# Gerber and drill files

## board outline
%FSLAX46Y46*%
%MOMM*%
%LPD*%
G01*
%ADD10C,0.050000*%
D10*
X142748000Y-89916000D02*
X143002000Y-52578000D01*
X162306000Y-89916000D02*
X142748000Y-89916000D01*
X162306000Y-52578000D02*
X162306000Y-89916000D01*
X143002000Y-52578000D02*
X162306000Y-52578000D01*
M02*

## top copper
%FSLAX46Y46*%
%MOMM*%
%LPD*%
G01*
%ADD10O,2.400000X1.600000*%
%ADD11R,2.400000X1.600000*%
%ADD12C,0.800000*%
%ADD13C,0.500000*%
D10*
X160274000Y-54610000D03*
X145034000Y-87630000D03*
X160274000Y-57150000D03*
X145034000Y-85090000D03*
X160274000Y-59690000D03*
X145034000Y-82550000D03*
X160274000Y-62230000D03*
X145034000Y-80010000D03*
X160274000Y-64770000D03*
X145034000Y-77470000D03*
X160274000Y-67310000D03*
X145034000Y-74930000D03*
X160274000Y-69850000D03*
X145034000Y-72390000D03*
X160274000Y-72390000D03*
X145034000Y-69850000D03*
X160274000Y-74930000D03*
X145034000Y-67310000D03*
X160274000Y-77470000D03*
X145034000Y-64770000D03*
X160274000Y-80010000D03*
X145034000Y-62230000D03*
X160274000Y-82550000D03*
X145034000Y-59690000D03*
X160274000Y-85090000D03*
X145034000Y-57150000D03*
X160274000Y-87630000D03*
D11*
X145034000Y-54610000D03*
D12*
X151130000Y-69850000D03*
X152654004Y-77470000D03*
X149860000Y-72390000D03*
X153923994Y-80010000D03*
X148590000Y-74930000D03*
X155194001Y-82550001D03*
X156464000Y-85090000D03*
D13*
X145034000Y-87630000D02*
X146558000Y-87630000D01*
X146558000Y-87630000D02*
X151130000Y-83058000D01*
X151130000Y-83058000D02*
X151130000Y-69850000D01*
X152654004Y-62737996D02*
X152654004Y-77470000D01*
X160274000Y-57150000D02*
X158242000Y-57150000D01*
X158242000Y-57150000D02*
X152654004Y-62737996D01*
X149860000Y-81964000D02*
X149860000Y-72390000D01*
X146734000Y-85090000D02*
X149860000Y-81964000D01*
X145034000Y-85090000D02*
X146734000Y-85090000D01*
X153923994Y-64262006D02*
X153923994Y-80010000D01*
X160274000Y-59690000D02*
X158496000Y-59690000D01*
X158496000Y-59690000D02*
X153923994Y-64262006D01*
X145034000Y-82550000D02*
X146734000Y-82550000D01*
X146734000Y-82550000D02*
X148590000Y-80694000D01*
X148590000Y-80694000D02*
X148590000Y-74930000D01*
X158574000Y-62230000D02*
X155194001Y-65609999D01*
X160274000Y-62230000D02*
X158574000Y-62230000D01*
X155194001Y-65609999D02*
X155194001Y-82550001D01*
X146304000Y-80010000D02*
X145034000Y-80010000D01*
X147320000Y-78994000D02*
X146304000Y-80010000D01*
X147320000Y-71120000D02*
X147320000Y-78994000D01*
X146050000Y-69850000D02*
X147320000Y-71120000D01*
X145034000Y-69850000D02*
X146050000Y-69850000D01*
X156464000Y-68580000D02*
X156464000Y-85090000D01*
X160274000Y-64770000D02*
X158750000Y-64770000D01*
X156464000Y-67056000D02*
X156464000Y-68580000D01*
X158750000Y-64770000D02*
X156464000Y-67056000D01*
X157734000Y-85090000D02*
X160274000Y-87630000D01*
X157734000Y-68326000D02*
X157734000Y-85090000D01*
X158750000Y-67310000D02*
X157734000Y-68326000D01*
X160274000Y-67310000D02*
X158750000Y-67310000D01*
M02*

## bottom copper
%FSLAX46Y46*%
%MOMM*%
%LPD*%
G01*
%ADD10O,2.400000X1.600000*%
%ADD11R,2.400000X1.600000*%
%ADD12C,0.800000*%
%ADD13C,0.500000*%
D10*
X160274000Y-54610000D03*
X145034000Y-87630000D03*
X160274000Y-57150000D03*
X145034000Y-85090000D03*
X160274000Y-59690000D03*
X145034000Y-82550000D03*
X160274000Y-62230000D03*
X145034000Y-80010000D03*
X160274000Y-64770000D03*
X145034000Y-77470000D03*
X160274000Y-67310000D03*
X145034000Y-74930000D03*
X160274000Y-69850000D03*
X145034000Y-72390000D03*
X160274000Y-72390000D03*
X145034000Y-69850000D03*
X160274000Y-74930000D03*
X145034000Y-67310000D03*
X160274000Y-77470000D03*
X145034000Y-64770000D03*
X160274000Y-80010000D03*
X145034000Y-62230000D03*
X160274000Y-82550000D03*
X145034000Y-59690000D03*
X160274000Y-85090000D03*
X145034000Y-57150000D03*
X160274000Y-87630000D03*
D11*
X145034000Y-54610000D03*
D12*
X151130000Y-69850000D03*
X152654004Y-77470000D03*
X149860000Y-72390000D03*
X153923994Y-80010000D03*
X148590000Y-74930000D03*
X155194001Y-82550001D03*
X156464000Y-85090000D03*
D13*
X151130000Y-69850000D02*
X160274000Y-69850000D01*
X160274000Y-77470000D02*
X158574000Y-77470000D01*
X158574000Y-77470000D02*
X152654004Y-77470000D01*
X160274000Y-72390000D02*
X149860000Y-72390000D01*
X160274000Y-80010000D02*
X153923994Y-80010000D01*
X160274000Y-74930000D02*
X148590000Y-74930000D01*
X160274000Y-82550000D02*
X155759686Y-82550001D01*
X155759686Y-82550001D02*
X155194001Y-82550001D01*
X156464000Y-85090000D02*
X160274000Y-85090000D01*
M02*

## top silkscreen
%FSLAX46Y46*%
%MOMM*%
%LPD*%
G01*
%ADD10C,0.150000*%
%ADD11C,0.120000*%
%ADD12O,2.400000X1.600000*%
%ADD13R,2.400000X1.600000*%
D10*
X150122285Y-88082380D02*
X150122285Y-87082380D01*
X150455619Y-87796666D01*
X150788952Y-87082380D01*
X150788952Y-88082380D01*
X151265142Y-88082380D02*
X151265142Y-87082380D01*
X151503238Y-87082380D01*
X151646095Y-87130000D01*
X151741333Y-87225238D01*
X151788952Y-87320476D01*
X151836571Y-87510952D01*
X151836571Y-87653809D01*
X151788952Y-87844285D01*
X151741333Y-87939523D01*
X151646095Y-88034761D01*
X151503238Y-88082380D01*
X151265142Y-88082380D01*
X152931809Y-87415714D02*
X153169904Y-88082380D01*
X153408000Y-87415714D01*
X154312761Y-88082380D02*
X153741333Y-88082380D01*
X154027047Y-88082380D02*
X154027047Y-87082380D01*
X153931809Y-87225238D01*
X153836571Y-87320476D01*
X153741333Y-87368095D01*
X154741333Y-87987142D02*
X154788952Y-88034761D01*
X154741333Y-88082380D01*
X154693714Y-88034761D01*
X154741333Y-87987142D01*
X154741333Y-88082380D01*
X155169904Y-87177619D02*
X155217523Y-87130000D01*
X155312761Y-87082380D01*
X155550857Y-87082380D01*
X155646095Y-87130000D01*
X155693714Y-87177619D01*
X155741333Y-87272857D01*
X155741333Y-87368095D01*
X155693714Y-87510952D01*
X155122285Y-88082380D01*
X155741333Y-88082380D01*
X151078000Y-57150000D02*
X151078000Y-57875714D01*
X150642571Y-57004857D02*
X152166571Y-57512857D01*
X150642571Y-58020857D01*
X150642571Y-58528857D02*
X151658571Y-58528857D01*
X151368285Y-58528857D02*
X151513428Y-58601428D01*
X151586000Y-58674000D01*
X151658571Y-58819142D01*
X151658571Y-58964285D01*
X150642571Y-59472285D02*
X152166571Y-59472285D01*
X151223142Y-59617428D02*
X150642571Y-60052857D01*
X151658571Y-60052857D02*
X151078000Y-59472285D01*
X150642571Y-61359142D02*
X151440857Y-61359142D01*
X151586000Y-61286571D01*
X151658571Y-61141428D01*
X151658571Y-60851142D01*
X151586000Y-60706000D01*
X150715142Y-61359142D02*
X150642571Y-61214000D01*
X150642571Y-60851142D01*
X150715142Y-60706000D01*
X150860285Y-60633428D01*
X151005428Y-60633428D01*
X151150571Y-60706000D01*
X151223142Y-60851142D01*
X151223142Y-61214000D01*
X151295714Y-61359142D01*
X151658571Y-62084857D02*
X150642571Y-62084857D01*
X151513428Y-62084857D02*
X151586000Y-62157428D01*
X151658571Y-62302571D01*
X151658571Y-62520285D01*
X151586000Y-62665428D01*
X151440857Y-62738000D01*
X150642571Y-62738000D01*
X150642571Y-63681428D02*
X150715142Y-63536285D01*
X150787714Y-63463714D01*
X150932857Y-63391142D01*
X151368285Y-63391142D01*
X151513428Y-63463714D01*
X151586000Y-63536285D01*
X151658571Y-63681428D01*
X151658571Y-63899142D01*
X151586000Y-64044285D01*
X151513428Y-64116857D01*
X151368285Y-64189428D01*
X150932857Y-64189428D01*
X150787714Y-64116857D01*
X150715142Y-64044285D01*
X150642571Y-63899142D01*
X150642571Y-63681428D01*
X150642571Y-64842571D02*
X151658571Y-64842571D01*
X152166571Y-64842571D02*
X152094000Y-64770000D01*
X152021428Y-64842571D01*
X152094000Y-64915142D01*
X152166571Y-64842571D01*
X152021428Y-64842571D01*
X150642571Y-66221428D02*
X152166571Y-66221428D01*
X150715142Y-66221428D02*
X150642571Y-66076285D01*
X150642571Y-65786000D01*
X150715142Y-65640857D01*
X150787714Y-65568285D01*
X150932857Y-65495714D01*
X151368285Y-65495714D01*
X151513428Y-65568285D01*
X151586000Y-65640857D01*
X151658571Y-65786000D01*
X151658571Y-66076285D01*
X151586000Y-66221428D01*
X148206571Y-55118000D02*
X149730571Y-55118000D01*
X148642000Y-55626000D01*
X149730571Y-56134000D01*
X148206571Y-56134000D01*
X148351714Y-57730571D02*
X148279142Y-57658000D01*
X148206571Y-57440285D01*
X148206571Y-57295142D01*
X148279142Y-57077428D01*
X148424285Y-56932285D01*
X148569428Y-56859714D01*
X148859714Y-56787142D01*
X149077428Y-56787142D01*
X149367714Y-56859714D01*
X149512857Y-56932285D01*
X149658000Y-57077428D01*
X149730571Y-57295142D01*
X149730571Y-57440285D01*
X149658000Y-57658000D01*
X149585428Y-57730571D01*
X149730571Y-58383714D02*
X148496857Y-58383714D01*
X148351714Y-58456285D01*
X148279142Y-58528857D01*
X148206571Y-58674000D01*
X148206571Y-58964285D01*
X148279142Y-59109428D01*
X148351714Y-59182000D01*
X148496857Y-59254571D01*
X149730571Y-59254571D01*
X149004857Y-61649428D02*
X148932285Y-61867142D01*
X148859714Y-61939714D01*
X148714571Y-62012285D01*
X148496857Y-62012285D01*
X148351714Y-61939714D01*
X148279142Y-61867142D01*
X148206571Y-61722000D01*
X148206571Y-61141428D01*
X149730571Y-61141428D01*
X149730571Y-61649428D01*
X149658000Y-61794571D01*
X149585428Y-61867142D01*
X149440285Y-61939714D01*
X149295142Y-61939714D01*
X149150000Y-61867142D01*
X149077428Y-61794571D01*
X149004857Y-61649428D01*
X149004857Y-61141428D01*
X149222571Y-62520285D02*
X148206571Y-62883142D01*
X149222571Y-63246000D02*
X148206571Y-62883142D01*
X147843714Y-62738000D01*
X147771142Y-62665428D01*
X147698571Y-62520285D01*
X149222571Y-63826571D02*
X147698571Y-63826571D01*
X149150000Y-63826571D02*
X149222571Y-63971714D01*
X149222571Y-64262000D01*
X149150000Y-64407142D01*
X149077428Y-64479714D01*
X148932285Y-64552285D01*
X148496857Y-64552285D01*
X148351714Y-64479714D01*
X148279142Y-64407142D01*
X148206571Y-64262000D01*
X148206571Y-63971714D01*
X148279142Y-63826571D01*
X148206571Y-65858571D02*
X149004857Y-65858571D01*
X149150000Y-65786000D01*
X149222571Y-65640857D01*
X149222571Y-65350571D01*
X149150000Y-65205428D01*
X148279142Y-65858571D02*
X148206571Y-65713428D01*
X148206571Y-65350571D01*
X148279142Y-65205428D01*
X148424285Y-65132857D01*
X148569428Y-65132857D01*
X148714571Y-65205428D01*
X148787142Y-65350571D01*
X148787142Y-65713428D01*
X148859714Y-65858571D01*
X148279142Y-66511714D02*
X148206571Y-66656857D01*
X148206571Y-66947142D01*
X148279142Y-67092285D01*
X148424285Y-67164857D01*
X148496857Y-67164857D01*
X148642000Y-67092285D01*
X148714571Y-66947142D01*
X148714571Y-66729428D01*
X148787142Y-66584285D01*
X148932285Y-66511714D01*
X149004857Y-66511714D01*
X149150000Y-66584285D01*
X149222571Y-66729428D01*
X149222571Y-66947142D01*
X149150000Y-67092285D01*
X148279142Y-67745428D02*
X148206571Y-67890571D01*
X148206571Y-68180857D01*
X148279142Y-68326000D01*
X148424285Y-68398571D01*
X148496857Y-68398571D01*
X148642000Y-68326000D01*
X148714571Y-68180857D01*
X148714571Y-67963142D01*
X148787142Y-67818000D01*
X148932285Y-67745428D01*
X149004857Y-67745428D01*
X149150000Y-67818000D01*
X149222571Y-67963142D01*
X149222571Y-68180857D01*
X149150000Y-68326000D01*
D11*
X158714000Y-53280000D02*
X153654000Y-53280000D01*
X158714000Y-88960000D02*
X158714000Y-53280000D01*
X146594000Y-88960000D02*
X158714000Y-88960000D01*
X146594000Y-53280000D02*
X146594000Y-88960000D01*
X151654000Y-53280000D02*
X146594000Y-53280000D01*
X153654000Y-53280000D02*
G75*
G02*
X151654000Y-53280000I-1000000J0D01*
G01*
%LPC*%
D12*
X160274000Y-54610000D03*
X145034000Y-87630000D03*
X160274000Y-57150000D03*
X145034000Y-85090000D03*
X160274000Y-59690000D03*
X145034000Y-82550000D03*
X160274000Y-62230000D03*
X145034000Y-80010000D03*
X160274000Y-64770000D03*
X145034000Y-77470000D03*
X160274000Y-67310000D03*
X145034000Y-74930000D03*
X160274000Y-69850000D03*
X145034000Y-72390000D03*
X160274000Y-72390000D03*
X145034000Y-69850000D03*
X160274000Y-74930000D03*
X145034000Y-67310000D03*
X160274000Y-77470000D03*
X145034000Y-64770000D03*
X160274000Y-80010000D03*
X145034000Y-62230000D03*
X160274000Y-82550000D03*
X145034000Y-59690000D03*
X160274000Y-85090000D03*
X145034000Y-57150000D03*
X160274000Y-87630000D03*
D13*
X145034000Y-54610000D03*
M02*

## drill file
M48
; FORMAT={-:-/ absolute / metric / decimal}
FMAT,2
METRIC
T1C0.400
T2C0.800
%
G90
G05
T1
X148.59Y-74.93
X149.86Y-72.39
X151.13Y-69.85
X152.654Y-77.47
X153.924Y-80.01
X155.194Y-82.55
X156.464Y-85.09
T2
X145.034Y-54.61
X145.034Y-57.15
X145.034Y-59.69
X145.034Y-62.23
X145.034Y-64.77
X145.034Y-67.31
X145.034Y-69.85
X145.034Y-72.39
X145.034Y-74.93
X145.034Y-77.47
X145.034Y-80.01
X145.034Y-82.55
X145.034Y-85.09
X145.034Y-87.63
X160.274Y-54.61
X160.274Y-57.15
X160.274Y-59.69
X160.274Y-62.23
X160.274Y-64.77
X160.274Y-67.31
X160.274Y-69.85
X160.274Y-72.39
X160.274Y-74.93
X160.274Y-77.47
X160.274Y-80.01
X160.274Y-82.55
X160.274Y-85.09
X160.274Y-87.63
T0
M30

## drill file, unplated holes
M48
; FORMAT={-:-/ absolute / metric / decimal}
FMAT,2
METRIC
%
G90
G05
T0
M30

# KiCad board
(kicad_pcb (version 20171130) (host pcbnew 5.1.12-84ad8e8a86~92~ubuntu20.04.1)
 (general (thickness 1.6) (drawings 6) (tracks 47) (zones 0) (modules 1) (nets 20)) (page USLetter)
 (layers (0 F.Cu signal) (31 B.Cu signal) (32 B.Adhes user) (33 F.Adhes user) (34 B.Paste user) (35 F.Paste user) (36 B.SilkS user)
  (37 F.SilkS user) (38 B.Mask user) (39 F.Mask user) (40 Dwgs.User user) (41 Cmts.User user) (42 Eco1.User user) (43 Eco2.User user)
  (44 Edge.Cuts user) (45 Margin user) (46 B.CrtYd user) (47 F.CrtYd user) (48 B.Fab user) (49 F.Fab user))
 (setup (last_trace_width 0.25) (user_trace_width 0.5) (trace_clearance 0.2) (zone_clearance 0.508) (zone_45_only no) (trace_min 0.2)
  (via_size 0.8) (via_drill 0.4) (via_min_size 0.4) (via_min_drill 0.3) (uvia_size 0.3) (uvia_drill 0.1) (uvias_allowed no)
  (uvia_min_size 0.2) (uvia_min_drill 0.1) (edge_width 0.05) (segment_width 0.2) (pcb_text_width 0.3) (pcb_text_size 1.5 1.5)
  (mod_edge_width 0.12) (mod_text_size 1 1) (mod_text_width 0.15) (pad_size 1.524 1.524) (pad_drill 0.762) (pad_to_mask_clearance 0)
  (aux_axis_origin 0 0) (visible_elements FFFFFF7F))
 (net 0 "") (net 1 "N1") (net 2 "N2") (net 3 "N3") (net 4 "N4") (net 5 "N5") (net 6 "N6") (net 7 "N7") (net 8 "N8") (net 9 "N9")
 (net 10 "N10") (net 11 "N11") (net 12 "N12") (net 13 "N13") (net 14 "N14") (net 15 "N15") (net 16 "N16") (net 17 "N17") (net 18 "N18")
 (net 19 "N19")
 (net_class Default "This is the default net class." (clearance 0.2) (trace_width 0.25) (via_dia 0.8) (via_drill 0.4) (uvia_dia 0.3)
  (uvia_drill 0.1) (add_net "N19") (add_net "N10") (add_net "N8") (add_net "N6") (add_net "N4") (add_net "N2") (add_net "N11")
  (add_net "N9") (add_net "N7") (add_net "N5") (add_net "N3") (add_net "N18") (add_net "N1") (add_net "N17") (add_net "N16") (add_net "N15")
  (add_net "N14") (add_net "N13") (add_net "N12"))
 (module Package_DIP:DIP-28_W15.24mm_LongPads (layer F.Cu) (at 145.034 54.61)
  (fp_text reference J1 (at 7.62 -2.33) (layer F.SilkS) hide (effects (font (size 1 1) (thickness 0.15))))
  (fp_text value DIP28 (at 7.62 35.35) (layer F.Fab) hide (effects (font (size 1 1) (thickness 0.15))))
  (fp_line (start 6.62 -1.33) (end 1.56 -1.33) (layer F.SilkS) (width 0.12))
  (fp_line (start 1.56 -1.33) (end 1.56 34.35) (layer F.SilkS) (width 0.12))
  (fp_line (start 1.56 34.35) (end 13.68 34.35) (layer F.SilkS) (width 0.12))
  (fp_line (start 13.68 34.35) (end 13.68 -1.33) (layer F.SilkS) (width 0.12))
  (fp_line (start 13.68 -1.33) (end 8.62 -1.33) (layer F.SilkS) (width 0.12))
  (fp_arc (start 7.62 -1.33) (end 6.62 -1.33) (angle -180) (layer F.SilkS) (width 0.12))
  (pad 28 thru_hole oval (at 15.24 0) (size 2.4 1.6) (drill 0.8) (layers *.Cu *.Mask) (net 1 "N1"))
  (pad 14 thru_hole oval (at 0 33.02) (size 2.4 1.6) (drill 0.8) (layers *.Cu *.Mask) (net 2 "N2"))
  (pad 27 thru_hole oval (at 15.24 2.54) (size 2.4 1.6) (drill 0.8) (layers *.Cu *.Mask) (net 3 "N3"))
  (pad 13 thru_hole oval (at 0 30.48) (size 2.4 1.6) (drill 0.8) (layers *.Cu *.Mask) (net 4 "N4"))
  (pad 26 thru_hole oval (at 15.24 5.08) (size 2.4 1.6) (drill 0.8) (layers *.Cu *.Mask) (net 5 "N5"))
  (pad 12 thru_hole oval (at 0 27.94) (size 2.4 1.6) (drill 0.8) (layers *.Cu *.Mask) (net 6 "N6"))
  (pad 25 thru_hole oval (at 15.24 7.62) (size 2.4 1.6) (drill 0.8) (layers *.Cu *.Mask) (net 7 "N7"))
  (pad 11 thru_hole oval (at 0 25.4) (size 2.4 1.6) (drill 0.8) (layers *.Cu *.Mask) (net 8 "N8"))
  (pad 24 thru_hole oval (at 15.24 10.16) (size 2.4 1.6) (drill 0.8) (layers *.Cu *.Mask) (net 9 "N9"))
  (pad 10 thru_hole oval (at 0 22.86) (size 2.4 1.6) (drill 0.8) (layers *.Cu *.Mask) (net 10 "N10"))
  (pad 23 thru_hole oval (at 15.24 12.7) (size 2.4 1.6) (drill 0.8) (layers *.Cu *.Mask) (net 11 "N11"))
  (pad 9 thru_hole oval (at 0 20.32) (size 2.4 1.6) (drill 0.8) (layers *.Cu *.Mask) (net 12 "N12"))
  (pad 22 thru_hole oval (at 15.24 15.24) (size 2.4 1.6) (drill 0.8) (layers *.Cu *.Mask) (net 2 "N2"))
  (pad 8 thru_hole oval (at 0 17.78) (size 2.4 1.6) (drill 0.8) (layers *.Cu *.Mask) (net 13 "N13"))
  (pad 21 thru_hole oval (at 15.24 17.78) (size 2.4 1.6) (drill 0.8) (layers *.Cu *.Mask) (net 4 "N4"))
  (pad 7 thru_hole oval (at 0 15.24) (size 2.4 1.6) (drill 0.8) (layers *.Cu *.Mask) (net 8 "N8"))
  (pad 20 thru_hole oval (at 15.24 20.32) (size 2.4 1.6) (drill 0.8) (layers *.Cu *.Mask) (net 6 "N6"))
  (pad 6 thru_hole oval (at 0 12.7) (size 2.4 1.6) (drill 0.8) (layers *.Cu *.Mask) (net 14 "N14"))
  (pad 19 thru_hole oval (at 15.24 22.86) (size 2.4 1.6) (drill 0.8) (layers *.Cu *.Mask) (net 3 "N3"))
  (pad 5 thru_hole oval (at 0 10.16) (size 2.4 1.6) (drill 0.8) (layers *.Cu *.Mask) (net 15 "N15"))
  (pad 18 thru_hole oval (at 15.24 25.4) (size 2.4 1.6) (drill 0.8) (layers *.Cu *.Mask) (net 5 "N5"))
  (pad 4 thru_hole oval (at 0 7.62) (size 2.4 1.6) (drill 0.8) (layers *.Cu *.Mask) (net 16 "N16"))
  (pad 17 thru_hole oval (at 15.24 27.94) (size 2.4 1.6) (drill 0.8) (layers *.Cu *.Mask) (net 7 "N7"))
  (pad 3 thru_hole oval (at 0 5.08) (size 2.4 1.6) (drill 0.8) (layers *.Cu *.Mask) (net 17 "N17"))
  (pad 16 thru_hole oval (at 15.24 30.48) (size 2.4 1.6) (drill 0.8) (layers *.Cu *.Mask) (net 9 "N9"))
  (pad 2 thru_hole oval (at 0 2.54) (size 2.4 1.6) (drill 0.8) (layers *.Cu *.Mask) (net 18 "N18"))
  (pad 15 thru_hole oval (at 15.24 33.02) (size 2.4 1.6) (drill 0.8) (layers *.Cu *.Mask) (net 11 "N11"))
  (pad 1 thru_hole rect (at 0 0) (size 2.4 1.6) (drill 0.8) (layers *.Cu *.Mask) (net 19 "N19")))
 (gr_line (start 142.748 89.916) (end 143.002 52.578) (layer Edge.Cuts) (width 0.05))
 (gr_line (start 162.306 89.916) (end 142.748 89.916) (layer Edge.Cuts) (width 0.05))
 (gr_line (start 162.306 52.578) (end 162.306 89.916) (layer Edge.Cuts) (width 0.05))
 (gr_line (start 143.002 52.578) (end 162.306 52.578) (layer Edge.Cuts) (width 0.05))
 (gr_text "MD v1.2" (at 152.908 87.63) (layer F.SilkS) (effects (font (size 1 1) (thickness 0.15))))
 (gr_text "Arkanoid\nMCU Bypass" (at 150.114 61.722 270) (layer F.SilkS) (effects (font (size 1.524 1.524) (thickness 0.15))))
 (segment (start 145.034 87.63) (end 146.558 87.63) (width 0.5) (layer F.Cu) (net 2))
 (segment (start 146.558 87.63) (end 151.13 83.058) (width 0.5) (layer F.Cu) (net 2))
 (segment (start 151.13 83.058) (end 151.13 69.85) (width 0.5) (layer F.Cu) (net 2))
 (via (at 151.13 69.85) (size 0.8) (drill 0.4) (layers F.Cu B.Cu) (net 2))
 (segment (start 151.13 69.85) (end 160.274 69.85) (width 0.5) (layer B.Cu) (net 2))
 (via (at 152.654004 77.47) (size 0.8) (drill 0.4) (layers F.Cu B.Cu) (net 3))
 (segment (start 160.274 77.47) (end 158.574 77.47) (width 0.5) (layer B.Cu) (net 3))
 (segment (start 152.654004 62.737996) (end 152.654004 77.47) (width 0.5) (layer F.Cu) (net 3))
 (segment (start 158.574 77.47) (end 152.654004 77.47) (width 0.5) (layer B.Cu) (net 3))
 (segment (start 160.274 57.15) (end 158.242 57.15) (width 0.5) (layer F.Cu) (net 3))
 (segment (start 158.242 57.15) (end 152.654004 62.737996) (width 0.5) (layer F.Cu) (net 3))
 (segment (start 149.86 81.964) (end 149.86 72.39) (width 0.5) (layer F.Cu) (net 4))
 (segment (start 146.734 85.09) (end 149.86 81.964) (width 0.5) (layer F.Cu) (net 4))
 (segment (start 145.034 85.09) (end 146.734 85.09) (width 0.5) (layer F.Cu) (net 4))
 (segment (start 160.274 72.39) (end 149.86 72.39) (width 0.5) (layer B.Cu) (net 4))
 (via (at 149.86 72.39) (size 0.8) (drill 0.4) (layers F.Cu B.Cu) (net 4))
 (via (at 153.923994 80.01) (size 0.8) (drill 0.4) (layers F.Cu B.Cu) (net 5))
 (segment (start 160.274 80.01) (end 153.923994 80.01) (width 0.5) (layer B.Cu) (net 5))
 (segment (start 153.923994 64.262006) (end 153.923994 80.01) (width 0.5) (layer F.Cu) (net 5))
 (segment (start 160.274 59.69) (end 158.496 59.69) (width 0.5) (layer F.Cu) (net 5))
 (segment (start 158.496 59.69) (end 153.923994 64.262006) (width 0.5) (layer F.Cu) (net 5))
 (via (at 148.59 74.93) (size 0.8) (drill 0.4) (layers F.Cu B.Cu) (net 6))
 (segment (start 160.274 74.93) (end 148.59 74.93) (width 0.5) (layer B.Cu) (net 6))
 (segment (start 145.034 82.55) (end 146.734 82.55) (width 0.5) (layer F.Cu) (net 6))
 (segment (start 146.734 82.55) (end 148.59 80.694) (width 0.5) (layer F.Cu) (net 6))
 (segment (start 148.59 80.694) (end 148.59 74.93) (width 0.5) (layer F.Cu) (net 6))
 (via (at 155.194001 82.550001) (size 0.8) (drill 0.4) (layers F.Cu B.Cu) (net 7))
 (segment (start 160.274 82.55) (end 155.759686 82.550001) (width 0.5) (layer B.Cu) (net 7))
 (segment (start 155.759686 82.550001) (end 155.194001 82.550001) (width 0.5) (layer B.Cu) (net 7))
 (segment (start 158.574 62.23) (end 155.194001 65.609999) (width 0.5) (layer F.Cu) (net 7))
 (segment (start 160.274 62.23) (end 158.574 62.23) (width 0.5) (layer F.Cu) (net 7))
 (segment (start 155.194001 65.609999) (end 155.194001 82.550001) (width 0.5) (layer F.Cu) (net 7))
 (segment (start 146.304 80.01) (end 145.034 80.01) (width 0.5) (layer F.Cu) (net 8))
 (segment (start 147.32 78.994) (end 146.304 80.01) (width 0.5) (layer F.Cu) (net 8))
 (segment (start 147.32 71.12) (end 147.32 78.994) (width 0.5) (layer F.Cu) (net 8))
 (segment (start 146.05 69.85) (end 147.32 71.12) (width 0.5) (layer F.Cu) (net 8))
 (segment (start 145.034 69.85) (end 146.05 69.85) (width 0.5) (layer F.Cu) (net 8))
 (segment (start 156.464 68.58) (end 156.464 85.09) (width 0.5) (layer F.Cu) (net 9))
 (via (at 156.464 85.09) (size 0.8) (drill 0.4) (layers F.Cu B.Cu) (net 9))
 (segment (start 156.464 85.09) (end 160.274 85.09) (width 0.5) (layer B.Cu) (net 9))
 (segment (start 160.274 64.77) (end 158.75 64.77) (width 0.5) (layer F.Cu) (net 9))
 (segment (start 156.464 67.056) (end 156.464 68.58) (width 0.5) (layer F.Cu) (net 9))
 (segment (start 158.75 64.77) (end 156.464 67.056) (width 0.5) (layer F.Cu) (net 9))
 (segment (start 157.734 85.09) (end 160.274 87.63) (width 0.5) (layer F.Cu) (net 11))
 (segment (start 157.734 68.326) (end 157.734 85.09) (width 0.5) (layer F.Cu) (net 11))
 (segment (start 158.75 67.31) (end 157.734 68.326) (width 0.5) (layer F.Cu) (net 11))
 (segment (start 160.274 67.31) (end 158.75 67.31) (width 0.5) (layer F.Cu) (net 11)))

